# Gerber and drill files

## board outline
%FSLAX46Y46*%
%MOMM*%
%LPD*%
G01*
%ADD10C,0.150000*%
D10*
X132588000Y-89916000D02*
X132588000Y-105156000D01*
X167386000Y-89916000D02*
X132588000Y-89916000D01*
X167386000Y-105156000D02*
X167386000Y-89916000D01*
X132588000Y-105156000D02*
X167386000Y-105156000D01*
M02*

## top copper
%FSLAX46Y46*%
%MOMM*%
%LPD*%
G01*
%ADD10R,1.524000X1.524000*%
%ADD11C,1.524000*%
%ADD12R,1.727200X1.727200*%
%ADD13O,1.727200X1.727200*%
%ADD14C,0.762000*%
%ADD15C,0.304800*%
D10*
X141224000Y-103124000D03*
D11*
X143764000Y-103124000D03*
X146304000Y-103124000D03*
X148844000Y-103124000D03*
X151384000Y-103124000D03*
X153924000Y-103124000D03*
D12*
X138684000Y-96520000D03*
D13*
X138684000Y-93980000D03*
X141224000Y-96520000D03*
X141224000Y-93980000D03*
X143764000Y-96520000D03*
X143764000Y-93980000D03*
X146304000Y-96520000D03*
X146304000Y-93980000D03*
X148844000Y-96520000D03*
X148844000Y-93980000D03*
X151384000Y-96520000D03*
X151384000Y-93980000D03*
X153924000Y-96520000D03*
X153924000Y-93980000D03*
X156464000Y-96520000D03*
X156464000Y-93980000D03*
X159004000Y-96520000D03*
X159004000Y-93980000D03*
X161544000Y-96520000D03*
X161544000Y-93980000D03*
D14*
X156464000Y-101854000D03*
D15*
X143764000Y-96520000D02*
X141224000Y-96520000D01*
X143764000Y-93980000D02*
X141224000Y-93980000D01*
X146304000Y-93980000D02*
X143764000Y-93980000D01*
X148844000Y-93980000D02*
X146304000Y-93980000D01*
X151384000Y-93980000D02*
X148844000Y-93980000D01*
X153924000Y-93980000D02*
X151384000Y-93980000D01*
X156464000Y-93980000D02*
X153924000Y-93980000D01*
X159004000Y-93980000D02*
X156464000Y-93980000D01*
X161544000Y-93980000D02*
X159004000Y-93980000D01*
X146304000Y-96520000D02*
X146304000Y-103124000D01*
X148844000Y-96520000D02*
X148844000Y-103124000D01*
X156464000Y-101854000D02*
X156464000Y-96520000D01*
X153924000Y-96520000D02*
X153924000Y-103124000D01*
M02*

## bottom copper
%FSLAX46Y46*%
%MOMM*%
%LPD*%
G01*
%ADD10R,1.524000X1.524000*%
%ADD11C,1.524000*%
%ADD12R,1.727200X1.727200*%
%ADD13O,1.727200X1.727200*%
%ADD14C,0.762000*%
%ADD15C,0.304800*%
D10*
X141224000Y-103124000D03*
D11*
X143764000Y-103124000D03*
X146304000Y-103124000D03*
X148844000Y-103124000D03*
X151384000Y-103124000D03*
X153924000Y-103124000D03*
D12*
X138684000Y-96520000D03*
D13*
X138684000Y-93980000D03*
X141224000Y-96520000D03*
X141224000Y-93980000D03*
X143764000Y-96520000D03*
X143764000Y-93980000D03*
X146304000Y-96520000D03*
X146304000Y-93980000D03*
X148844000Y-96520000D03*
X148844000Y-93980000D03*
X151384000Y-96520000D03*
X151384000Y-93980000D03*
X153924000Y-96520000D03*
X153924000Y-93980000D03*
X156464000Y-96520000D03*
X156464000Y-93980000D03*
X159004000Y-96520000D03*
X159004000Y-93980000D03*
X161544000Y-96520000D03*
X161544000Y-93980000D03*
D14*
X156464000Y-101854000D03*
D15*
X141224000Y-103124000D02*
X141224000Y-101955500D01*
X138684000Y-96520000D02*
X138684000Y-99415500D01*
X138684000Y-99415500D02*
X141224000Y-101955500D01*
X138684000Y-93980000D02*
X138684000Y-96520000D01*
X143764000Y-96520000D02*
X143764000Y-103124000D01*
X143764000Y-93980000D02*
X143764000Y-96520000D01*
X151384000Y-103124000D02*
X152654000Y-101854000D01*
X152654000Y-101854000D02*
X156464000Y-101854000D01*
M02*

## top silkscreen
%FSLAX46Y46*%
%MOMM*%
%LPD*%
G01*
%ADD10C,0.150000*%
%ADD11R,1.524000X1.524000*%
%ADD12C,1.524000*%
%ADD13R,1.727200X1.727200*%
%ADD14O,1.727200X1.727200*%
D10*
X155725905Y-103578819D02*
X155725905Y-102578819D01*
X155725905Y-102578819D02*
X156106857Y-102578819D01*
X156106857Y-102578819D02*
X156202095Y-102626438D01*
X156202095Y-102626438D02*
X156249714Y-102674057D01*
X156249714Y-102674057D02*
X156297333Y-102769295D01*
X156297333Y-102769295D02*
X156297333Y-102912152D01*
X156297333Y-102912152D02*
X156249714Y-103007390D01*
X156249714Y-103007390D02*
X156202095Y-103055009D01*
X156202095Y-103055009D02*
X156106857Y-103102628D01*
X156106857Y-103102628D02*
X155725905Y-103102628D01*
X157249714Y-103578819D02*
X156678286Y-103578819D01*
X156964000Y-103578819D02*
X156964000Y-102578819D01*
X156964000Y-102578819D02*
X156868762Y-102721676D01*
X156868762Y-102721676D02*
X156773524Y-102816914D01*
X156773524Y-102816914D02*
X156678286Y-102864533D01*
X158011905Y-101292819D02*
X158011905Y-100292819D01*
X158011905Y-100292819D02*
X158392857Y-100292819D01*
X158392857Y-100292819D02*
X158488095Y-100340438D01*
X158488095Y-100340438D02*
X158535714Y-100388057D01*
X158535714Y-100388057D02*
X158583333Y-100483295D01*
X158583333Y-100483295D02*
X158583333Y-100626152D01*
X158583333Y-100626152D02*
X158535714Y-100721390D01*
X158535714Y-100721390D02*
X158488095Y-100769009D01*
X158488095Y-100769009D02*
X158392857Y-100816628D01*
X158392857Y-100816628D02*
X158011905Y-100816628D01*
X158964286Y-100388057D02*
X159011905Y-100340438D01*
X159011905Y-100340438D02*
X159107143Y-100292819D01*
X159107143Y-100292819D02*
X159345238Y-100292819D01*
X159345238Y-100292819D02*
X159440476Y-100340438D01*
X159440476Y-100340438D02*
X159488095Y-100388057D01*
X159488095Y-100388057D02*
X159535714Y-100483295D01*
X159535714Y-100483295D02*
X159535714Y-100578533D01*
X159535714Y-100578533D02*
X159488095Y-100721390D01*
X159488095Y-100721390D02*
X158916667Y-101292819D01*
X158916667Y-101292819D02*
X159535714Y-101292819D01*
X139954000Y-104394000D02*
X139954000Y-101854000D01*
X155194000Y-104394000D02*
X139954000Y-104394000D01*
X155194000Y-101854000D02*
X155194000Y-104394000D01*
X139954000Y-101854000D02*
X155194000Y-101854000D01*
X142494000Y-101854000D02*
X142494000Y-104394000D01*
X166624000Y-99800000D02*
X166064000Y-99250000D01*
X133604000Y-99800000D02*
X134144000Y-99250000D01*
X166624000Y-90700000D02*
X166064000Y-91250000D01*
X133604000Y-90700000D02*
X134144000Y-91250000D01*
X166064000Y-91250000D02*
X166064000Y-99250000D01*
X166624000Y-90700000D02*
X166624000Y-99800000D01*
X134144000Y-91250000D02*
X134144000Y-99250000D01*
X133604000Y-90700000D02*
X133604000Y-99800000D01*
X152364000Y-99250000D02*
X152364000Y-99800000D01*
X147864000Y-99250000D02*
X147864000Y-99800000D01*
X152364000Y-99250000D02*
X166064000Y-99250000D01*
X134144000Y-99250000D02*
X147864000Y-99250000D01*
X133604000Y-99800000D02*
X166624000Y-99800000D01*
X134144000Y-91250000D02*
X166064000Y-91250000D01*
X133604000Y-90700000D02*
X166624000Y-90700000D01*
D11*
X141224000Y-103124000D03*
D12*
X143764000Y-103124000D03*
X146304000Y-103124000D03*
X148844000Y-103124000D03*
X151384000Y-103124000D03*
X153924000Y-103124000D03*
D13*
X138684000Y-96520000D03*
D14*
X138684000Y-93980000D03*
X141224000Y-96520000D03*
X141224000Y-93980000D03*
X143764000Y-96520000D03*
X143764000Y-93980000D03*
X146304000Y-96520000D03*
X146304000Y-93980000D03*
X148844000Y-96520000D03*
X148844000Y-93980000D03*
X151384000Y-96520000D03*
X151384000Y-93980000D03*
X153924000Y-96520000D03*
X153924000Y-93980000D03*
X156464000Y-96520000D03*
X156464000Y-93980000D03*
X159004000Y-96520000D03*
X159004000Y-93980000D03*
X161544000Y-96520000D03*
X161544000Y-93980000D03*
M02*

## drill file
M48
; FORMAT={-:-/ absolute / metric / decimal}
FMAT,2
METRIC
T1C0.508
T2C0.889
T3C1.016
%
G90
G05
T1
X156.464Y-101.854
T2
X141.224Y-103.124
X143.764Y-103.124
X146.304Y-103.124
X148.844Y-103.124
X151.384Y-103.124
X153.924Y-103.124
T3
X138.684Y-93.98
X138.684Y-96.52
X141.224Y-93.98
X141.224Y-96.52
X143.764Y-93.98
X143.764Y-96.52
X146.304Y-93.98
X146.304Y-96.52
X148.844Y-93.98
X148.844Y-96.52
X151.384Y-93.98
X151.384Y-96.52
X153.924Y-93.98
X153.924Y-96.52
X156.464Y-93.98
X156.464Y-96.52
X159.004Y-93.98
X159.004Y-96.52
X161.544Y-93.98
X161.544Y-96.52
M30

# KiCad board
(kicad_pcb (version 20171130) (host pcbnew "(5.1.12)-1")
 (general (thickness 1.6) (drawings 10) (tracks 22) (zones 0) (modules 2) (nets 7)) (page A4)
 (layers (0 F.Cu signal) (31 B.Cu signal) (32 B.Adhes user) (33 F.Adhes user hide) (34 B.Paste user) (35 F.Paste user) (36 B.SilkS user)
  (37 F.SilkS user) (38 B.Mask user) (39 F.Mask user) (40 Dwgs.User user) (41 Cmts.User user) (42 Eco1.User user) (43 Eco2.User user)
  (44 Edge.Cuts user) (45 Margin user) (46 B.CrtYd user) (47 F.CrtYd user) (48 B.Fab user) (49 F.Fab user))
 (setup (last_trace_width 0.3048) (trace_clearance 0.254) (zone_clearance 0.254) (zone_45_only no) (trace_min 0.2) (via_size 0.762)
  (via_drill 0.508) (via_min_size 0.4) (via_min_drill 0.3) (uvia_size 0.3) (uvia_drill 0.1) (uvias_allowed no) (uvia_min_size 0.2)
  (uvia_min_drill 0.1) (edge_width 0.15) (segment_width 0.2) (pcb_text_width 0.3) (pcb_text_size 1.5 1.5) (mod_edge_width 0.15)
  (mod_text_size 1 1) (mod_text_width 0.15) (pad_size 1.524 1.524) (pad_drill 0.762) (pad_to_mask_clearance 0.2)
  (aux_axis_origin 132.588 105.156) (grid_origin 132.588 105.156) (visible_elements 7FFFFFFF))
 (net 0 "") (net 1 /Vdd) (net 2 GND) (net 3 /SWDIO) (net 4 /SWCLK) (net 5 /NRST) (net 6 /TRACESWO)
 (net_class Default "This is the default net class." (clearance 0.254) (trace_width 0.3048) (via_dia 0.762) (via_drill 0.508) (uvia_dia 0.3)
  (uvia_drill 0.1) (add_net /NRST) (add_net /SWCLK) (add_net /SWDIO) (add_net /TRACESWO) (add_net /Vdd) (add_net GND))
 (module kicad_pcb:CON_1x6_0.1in (layer F.Cu) (at 147.574 103.124)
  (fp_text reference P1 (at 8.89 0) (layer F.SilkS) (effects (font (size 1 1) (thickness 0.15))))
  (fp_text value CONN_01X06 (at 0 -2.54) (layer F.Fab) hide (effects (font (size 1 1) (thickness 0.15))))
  (fp_line (start -7.62 1.27) (end -7.62 -1.27) (layer F.SilkS) (width 0.15))
  (fp_line (start 7.62 1.27) (end -7.62 1.27) (layer F.SilkS) (width 0.15))
  (fp_line (start 7.62 -1.27) (end 7.62 1.27) (layer F.SilkS) (width 0.15))
  (fp_line (start -7.62 -1.27) (end 7.62 -1.27) (layer F.SilkS) (width 0.15))
  (fp_line (start -5.08 -1.27) (end -5.08 1.27) (layer F.SilkS) (width 0.15))
  (pad 1 thru_hole rect (at -6.35 0) (size 1.524 1.524) (drill 0.889) (layers *.Cu *.Mask F.SilkS) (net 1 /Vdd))
  (pad 2 thru_hole circle (at -3.81 0) (size 1.524 1.524) (drill 0.889) (layers *.Cu *.Mask F.SilkS) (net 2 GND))
  (pad 3 thru_hole circle (at -1.27 0) (size 1.524 1.524) (drill 0.889) (layers *.Cu *.Mask F.SilkS) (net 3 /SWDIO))
  (pad 4 thru_hole circle (at 1.27 0) (size 1.524 1.524) (drill 0.889) (layers *.Cu *.Mask F.SilkS) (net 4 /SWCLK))
  (pad 5 thru_hole circle (at 3.81 0) (size 1.524 1.524) (drill 0.889) (layers *.Cu *.Mask F.SilkS) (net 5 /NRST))
  (pad 6 thru_hole circle (at 6.35 0) (size 1.524 1.524) (drill 0.889) (layers *.Cu *.Mask F.SilkS) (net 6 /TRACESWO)))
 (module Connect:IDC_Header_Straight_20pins (layer F.Cu) (at 138.684 96.52)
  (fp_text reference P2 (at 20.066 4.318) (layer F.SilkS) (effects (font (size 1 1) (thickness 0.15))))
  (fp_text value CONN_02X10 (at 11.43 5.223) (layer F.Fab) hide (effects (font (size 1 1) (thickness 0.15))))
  (fp_line (start 27.94 3.28) (end 27.38 2.73) (layer F.SilkS) (width 0.15))
  (fp_line (start -5.08 3.28) (end -4.54 2.73) (layer F.SilkS) (width 0.15))
  (fp_line (start 27.94 -5.82) (end 27.38 -5.27) (layer F.SilkS) (width 0.15))
  (fp_line (start -5.08 -5.82) (end -4.54 -5.27) (layer F.SilkS) (width 0.15))
  (fp_line (start 27.38 -5.27) (end 27.38 2.73) (layer F.SilkS) (width 0.15))
  (fp_line (start 27.94 -5.82) (end 27.94 3.28) (layer F.SilkS) (width 0.15))
  (fp_line (start -4.54 -5.27) (end -4.54 2.73) (layer F.SilkS) (width 0.15))
  (fp_line (start -5.08 -5.82) (end -5.08 3.28) (layer F.SilkS) (width 0.15))
  (fp_line (start 13.68 2.73) (end 13.68 3.28) (layer F.SilkS) (width 0.15))
  (fp_line (start 9.18 2.73) (end 9.18 3.28) (layer F.SilkS) (width 0.15))
  (fp_line (start 13.68 2.73) (end 27.38 2.73) (layer F.SilkS) (width 0.15))
  (fp_line (start -4.54 2.73) (end 9.18 2.73) (layer F.SilkS) (width 0.15))
  (fp_line (start -5.08 3.28) (end 27.94 3.28) (layer F.SilkS) (width 0.15))
  (fp_line (start -4.54 -5.27) (end 27.38 -5.27) (layer F.SilkS) (width 0.15))
  (fp_line (start -5.08 -5.82) (end 27.94 -5.82) (layer F.SilkS) (width 0.15))
  (pad 1 thru_hole rect (at 0 0) (size 1.7272 1.7272) (drill 1.016) (layers *.Cu *.Mask F.SilkS) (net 1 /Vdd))
  (pad 2 thru_hole oval (at 0 -2.54) (size 1.7272 1.7272) (drill 1.016) (layers *.Cu *.Mask F.SilkS) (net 1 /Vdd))
  (pad 3 thru_hole oval (at 2.54 0) (size 1.7272 1.7272) (drill 1.016) (layers *.Cu *.Mask F.SilkS) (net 2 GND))
  (pad 4 thru_hole oval (at 2.54 -2.54) (size 1.7272 1.7272) (drill 1.016) (layers *.Cu *.Mask F.SilkS) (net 2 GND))
  (pad 5 thru_hole oval (at 5.08 0) (size 1.7272 1.7272) (drill 1.016) (layers *.Cu *.Mask F.SilkS) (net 2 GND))
  (pad 6 thru_hole oval (at 5.08 -2.54) (size 1.7272 1.7272) (drill 1.016) (layers *.Cu *.Mask F.SilkS) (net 2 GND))
  (pad 7 thru_hole oval (at 7.62 0) (size 1.7272 1.7272) (drill 1.016) (layers *.Cu *.Mask F.SilkS) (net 3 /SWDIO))
  (pad 8 thru_hole oval (at 7.62 -2.54) (size 1.7272 1.7272) (drill 1.016) (layers *.Cu *.Mask F.SilkS) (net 2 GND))
  (pad 9 thru_hole oval (at 10.16 0) (size 1.7272 1.7272) (drill 1.016) (layers *.Cu *.Mask F.SilkS) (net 4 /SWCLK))
  (pad 10 thru_hole oval (at 10.16 -2.54) (size 1.7272 1.7272) (drill 1.016) (layers *.Cu *.Mask F.SilkS) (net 2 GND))
  (pad 11 thru_hole oval (at 12.7 0) (size 1.7272 1.7272) (drill 1.016) (layers *.Cu *.Mask F.SilkS))
  (pad 12 thru_hole oval (at 12.7 -2.54) (size 1.7272 1.7272) (drill 1.016) (layers *.Cu *.Mask F.SilkS) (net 2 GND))
  (pad 13 thru_hole oval (at 15.24 0) (size 1.7272 1.7272) (drill 1.016) (layers *.Cu *.Mask F.SilkS) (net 6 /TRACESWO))
  (pad 14 thru_hole oval (at 15.24 -2.54) (size 1.7272 1.7272) (drill 1.016) (layers *.Cu *.Mask F.SilkS) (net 2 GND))
  (pad 15 thru_hole oval (at 17.78 0) (size 1.7272 1.7272) (drill 1.016) (layers *.Cu *.Mask F.SilkS) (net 5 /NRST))
  (pad 16 thru_hole oval (at 17.78 -2.54) (size 1.7272 1.7272) (drill 1.016) (layers *.Cu *.Mask F.SilkS) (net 2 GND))
  (pad 17 thru_hole oval (at 20.32 0) (size 1.7272 1.7272) (drill 1.016) (layers *.Cu *.Mask F.SilkS))
  (pad 18 thru_hole oval (at 20.32 -2.54) (size 1.7272 1.7272) (drill 1.016) (layers *.Cu *.Mask F.SilkS) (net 2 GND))
  (pad 19 thru_hole oval (at 22.86 0) (size 1.7272 1.7272) (drill 1.016) (layers *.Cu *.Mask F.SilkS))
  (pad 20 thru_hole oval (at 22.86 -2.54) (size 1.7272 1.7272) (drill 1.016) (layers *.Cu *.Mask F.SilkS) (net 2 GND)))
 (gr_line (start 132.588 89.916) (end 132.588 105.156) (angle 90) (layer Edge.Cuts) (width 0.15))
 (gr_line (start 167.386 89.916) (end 132.588 89.916) (angle 90) (layer Edge.Cuts) (width 0.15))
 (gr_line (start 167.386 105.156) (end 167.386 89.916) (angle 90) (layer Edge.Cuts) (width 0.15))
 (gr_line (start 132.588 105.156) (end 167.386 105.156) (angle 90) (layer Edge.Cuts) (width 0.15))
 (segment (start 141.224 103.124) (end 141.224 101.9555) (width 0.3048) (layer B.Cu) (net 1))
 (segment (start 138.684 96.52) (end 138.684 99.4155) (width 0.3048) (layer B.Cu) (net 1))
 (segment (start 138.684 99.4155) (end 141.224 101.9555) (width 0.3048) (layer B.Cu) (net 1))
 (segment (start 138.684 93.98) (end 138.684 96.52) (width 0.3048) (layer B.Cu) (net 1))
 (segment (start 143.764 96.52) (end 143.764 103.124) (width 0.3048) (layer B.Cu) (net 2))
 (segment (start 143.764 93.98) (end 143.764 96.52) (width 0.3048) (layer B.Cu) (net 2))
 (segment (start 143.764 96.52) (end 141.224 96.52) (width 0.3048) (layer F.Cu) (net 2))
 (segment (start 143.764 93.98) (end 141.224 93.98) (width 0.3048) (layer F.Cu) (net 2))
 (segment (start 146.304 93.98) (end 143.764 93.98) (width 0.3048) (layer F.Cu) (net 2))
 (segment (start 148.844 93.98) (end 146.304 93.98) (width 0.3048) (layer F.Cu) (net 2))
 (segment (start 151.384 93.98) (end 148.844 93.98) (width 0.3048) (layer F.Cu) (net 2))
 (segment (start 153.924 93.98) (end 151.384 93.98) (width 0.3048) (layer F.Cu) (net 2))
 (segment (start 156.464 93.98) (end 153.924 93.98) (width 0.3048) (layer F.Cu) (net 2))
 (segment (start 159.004 93.98) (end 156.464 93.98) (width 0.3048) (layer F.Cu) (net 2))
 (segment (start 161.544 93.98) (end 159.004 93.98) (width 0.3048) (layer F.Cu) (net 2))
 (segment (start 146.304 96.52) (end 146.304 103.124) (width 0.3048) (layer F.Cu) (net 3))
 (segment (start 148.844 96.52) (end 148.844 103.124) (width 0.3048) (layer F.Cu) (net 4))
 (segment (start 151.384 103.124) (end 152.654 101.854) (width 0.3048) (layer B.Cu) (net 5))
 (segment (start 152.654 101.854) (end 156.464 101.854) (width 0.3048) (layer B.Cu) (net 5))
 (segment (start 156.464 101.854) (end 156.464 96.52) (width 0.3048) (layer F.Cu) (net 5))
 (via (at 156.464 101.854) (size 0.762) (layers F.Cu B.Cu) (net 5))
 (segment (start 153.924 96.52) (end 153.924 103.124) (width 0.3048) (layer F.Cu) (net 6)))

